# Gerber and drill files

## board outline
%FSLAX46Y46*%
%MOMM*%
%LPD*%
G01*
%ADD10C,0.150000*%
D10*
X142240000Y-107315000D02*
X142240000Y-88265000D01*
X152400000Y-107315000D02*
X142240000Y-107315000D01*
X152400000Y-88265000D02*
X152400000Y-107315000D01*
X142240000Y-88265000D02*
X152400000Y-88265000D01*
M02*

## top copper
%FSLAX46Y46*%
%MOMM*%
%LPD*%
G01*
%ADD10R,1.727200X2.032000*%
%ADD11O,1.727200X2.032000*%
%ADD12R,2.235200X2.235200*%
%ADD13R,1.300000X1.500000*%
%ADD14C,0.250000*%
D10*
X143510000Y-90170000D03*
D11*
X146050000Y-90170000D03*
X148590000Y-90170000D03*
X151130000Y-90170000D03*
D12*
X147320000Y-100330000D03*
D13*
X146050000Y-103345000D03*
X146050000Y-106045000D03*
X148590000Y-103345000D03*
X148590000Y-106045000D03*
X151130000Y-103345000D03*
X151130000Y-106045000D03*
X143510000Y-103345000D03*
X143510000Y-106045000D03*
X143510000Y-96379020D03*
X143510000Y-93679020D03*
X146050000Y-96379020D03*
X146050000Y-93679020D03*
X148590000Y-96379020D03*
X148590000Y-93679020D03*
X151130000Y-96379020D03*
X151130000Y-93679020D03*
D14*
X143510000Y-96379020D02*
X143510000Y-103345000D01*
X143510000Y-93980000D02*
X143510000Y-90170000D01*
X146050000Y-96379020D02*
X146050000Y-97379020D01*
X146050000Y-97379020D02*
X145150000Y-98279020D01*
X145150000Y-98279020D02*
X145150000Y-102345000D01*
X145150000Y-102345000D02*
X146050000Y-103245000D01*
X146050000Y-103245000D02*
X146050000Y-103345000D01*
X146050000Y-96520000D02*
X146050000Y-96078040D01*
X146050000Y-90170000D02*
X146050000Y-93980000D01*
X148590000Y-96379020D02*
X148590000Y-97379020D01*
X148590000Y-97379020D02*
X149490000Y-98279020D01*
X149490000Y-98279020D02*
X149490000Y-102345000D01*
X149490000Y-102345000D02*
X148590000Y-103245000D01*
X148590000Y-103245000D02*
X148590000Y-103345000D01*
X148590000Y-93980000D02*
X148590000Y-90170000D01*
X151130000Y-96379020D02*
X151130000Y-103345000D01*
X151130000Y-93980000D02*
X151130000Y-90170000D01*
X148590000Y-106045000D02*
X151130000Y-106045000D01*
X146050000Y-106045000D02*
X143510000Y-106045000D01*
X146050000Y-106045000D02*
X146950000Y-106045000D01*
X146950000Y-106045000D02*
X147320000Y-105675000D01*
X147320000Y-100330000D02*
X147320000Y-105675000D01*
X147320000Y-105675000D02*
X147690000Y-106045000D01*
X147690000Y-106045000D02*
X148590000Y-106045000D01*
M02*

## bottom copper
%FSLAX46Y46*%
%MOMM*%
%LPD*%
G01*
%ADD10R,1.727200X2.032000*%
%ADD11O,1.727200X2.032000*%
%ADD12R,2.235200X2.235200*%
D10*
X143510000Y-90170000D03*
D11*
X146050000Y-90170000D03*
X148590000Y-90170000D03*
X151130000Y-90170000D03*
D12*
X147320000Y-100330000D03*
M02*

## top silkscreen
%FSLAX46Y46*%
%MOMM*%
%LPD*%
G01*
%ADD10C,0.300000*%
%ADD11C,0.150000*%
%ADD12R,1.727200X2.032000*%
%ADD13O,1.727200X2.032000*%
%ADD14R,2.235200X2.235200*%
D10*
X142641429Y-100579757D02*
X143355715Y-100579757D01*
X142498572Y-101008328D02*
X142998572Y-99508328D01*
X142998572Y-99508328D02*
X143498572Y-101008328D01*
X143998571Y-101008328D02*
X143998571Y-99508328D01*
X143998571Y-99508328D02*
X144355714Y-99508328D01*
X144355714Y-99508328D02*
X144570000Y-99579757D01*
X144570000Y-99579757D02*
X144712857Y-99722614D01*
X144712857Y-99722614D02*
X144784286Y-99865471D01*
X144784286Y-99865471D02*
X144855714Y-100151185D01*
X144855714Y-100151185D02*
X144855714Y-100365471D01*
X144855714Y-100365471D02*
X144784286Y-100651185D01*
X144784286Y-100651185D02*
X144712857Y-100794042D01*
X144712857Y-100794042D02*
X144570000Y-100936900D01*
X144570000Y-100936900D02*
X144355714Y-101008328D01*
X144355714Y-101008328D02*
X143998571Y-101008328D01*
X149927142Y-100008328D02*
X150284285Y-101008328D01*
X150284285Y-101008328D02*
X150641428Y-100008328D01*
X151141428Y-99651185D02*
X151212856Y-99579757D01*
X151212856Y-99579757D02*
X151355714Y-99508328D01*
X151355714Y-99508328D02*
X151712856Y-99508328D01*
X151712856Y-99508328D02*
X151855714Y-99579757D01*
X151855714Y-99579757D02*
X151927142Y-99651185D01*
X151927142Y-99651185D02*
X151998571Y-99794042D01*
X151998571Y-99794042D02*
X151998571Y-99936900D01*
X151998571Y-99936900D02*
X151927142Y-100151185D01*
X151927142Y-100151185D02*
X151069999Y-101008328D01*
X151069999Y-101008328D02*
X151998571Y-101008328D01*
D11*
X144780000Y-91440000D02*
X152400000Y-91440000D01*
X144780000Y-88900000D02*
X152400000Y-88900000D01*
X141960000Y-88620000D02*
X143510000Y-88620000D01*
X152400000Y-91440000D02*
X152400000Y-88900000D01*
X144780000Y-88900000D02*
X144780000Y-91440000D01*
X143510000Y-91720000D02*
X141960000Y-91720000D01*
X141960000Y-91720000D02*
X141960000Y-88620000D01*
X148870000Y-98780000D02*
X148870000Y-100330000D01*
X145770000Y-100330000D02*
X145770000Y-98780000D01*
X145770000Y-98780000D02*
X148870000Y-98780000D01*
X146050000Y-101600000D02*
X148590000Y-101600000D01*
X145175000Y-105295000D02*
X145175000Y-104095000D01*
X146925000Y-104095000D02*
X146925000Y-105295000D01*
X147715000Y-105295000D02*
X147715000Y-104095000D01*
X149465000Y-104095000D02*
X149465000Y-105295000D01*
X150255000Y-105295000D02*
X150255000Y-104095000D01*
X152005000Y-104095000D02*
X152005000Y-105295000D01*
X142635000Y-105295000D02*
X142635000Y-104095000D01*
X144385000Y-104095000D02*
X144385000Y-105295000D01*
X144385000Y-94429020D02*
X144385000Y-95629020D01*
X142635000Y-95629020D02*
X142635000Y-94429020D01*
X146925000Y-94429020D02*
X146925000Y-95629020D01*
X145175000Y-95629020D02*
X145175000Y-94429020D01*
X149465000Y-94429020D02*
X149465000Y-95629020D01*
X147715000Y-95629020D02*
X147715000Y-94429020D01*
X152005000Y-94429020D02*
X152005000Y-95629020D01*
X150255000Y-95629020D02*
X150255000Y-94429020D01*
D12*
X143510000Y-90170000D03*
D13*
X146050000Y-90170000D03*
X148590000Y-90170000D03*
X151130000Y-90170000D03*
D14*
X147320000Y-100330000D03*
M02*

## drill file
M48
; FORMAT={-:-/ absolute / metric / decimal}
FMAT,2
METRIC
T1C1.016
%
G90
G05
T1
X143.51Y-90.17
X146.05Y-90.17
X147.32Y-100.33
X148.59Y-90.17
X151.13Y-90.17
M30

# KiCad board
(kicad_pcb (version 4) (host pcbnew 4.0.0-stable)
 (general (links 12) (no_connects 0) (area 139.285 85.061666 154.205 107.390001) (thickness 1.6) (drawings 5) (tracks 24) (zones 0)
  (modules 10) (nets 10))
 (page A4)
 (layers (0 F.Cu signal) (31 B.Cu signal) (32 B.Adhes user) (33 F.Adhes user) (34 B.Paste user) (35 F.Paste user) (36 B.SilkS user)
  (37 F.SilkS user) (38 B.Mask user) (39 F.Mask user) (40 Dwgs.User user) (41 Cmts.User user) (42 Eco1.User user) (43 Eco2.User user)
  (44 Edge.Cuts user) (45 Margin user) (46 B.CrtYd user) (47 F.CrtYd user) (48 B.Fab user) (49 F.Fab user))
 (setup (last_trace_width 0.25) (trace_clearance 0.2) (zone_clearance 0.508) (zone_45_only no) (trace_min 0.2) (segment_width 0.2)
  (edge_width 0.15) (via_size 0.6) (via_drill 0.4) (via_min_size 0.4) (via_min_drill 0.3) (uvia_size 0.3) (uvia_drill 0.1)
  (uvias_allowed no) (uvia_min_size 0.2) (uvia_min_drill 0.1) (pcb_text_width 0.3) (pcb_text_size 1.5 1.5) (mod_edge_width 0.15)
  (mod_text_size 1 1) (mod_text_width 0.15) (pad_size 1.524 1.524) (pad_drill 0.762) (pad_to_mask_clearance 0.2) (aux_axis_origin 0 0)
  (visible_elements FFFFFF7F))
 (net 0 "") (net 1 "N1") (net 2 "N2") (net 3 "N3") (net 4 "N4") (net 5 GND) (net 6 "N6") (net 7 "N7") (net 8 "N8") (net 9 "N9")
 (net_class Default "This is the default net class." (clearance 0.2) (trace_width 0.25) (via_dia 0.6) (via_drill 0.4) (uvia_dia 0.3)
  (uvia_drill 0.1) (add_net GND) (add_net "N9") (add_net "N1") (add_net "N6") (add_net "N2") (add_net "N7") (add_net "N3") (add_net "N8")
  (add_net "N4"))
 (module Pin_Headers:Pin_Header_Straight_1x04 (layer F.Cu) (at 143.51 90.17 90)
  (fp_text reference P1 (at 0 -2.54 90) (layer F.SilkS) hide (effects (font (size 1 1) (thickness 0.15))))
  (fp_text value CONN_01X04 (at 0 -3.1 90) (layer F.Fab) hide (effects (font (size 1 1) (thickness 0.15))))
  (fp_line (start -1.27 1.27) (end -1.27 8.89) (layer F.SilkS) (width 0.15))
  (fp_line (start 1.27 1.27) (end 1.27 8.89) (layer F.SilkS) (width 0.15))
  (fp_line (start 1.55 -1.55) (end 1.55 0) (layer F.SilkS) (width 0.15))
  (fp_line (start -1.27 8.89) (end 1.27 8.89) (layer F.SilkS) (width 0.15))
  (fp_line (start 1.27 1.27) (end -1.27 1.27) (layer F.SilkS) (width 0.15))
  (fp_line (start -1.55 0) (end -1.55 -1.55) (layer F.SilkS) (width 0.15))
  (fp_line (start -1.55 -1.55) (end 1.55 -1.55) (layer F.SilkS) (width 0.15))
  (pad 1 thru_hole rect (at 0 0 90) (size 2.032 1.7272) (drill 1.016) (layers *.Cu *.Mask F.SilkS) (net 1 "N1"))
  (pad 2 thru_hole oval (at 0 2.54 90) (size 2.032 1.7272) (drill 1.016) (layers *.Cu *.Mask F.SilkS) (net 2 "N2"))
  (pad 3 thru_hole oval (at 0 5.08 90) (size 2.032 1.7272) (drill 1.016) (layers *.Cu *.Mask F.SilkS) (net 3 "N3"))
  (pad 4 thru_hole oval (at 0 7.62 90) (size 2.032 1.7272) (drill 1.016) (layers *.Cu *.Mask F.SilkS) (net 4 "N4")))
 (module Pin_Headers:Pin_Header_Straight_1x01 (layer F.Cu) (at 147.32 100.33)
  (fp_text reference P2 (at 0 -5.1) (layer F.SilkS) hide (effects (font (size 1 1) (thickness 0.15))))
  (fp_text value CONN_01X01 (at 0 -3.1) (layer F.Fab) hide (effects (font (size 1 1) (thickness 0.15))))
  (fp_line (start 1.55 -1.55) (end 1.55 0) (layer F.SilkS) (width 0.15))
  (fp_line (start -1.55 0) (end -1.55 -1.55) (layer F.SilkS) (width 0.15))
  (fp_line (start -1.55 -1.55) (end 1.55 -1.55) (layer F.SilkS) (width 0.15))
  (fp_line (start -1.27 1.27) (end 1.27 1.27) (layer F.SilkS) (width 0.15))
  (pad 1 thru_hole rect (at 0 0) (size 2.2352 2.2352) (drill 1.016) (layers *.Cu *.Mask F.SilkS) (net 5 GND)))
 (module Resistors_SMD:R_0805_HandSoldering (layer F.Cu) (at 146.05 104.695 270)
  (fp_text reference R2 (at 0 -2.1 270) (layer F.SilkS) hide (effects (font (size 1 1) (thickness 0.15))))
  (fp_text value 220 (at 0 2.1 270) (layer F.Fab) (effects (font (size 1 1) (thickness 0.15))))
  (fp_line (start 0.6 0.875) (end -0.6 0.875) (layer F.SilkS) (width 0.15))
  (fp_line (start -0.6 -0.875) (end 0.6 -0.875) (layer F.SilkS) (width 0.15))
  (pad 1 smd rect (at -1.35 0 270) (size 1.5 1.3) (layers F.Cu F.Paste F.Mask) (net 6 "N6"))
  (pad 2 smd rect (at 1.35 0 270) (size 1.5 1.3) (layers F.Cu F.Paste F.Mask) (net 5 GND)))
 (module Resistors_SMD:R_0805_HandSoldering (layer F.Cu) (at 148.59 104.695 270)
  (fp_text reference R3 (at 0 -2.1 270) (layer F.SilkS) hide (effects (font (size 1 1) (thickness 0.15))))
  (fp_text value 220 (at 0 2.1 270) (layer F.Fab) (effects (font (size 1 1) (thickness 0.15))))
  (fp_line (start 0.6 0.875) (end -0.6 0.875) (layer F.SilkS) (width 0.15))
  (fp_line (start -0.6 -0.875) (end 0.6 -0.875) (layer F.SilkS) (width 0.15))
  (pad 1 smd rect (at -1.35 0 270) (size 1.5 1.3) (layers F.Cu F.Paste F.Mask) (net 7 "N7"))
  (pad 2 smd rect (at 1.35 0 270) (size 1.5 1.3) (layers F.Cu F.Paste F.Mask) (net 5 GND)))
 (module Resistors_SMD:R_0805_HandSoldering (layer F.Cu) (at 151.13 104.695 270)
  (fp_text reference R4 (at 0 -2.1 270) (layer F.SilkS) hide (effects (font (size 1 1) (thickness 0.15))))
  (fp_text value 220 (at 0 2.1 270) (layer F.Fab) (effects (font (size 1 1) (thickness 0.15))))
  (fp_line (start 0.6 0.875) (end -0.6 0.875) (layer F.SilkS) (width 0.15))
  (fp_line (start -0.6 -0.875) (end 0.6 -0.875) (layer F.SilkS) (width 0.15))
  (pad 1 smd rect (at -1.35 0 270) (size 1.5 1.3) (layers F.Cu F.Paste F.Mask) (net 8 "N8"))
  (pad 2 smd rect (at 1.35 0 270) (size 1.5 1.3) (layers F.Cu F.Paste F.Mask) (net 5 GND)))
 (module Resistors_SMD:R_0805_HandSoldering (layer F.Cu) (at 143.51 104.695 270)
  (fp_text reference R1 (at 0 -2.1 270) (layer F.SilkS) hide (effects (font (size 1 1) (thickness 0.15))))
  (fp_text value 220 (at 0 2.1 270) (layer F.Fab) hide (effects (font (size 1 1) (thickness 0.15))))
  (fp_line (start 0.6 0.875) (end -0.6 0.875) (layer F.SilkS) (width 0.15))
  (fp_line (start -0.6 -0.875) (end 0.6 -0.875) (layer F.SilkS) (width 0.15))
  (pad 1 smd rect (at -1.35 0 270) (size 1.5 1.3) (layers F.Cu F.Paste F.Mask) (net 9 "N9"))
  (pad 2 smd rect (at 1.35 0 270) (size 1.5 1.3) (layers F.Cu F.Paste F.Mask) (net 5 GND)))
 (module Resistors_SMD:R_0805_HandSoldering (layer F.Cu) (at 143.51 95.02902 90)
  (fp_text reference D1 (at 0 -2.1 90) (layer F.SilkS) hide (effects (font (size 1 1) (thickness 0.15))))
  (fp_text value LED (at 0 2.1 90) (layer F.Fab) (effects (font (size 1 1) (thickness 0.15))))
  (fp_line (start 0.6 0.875) (end -0.6 0.875) (layer F.SilkS) (width 0.15))
  (fp_line (start -0.6 -0.875) (end 0.6 -0.875) (layer F.SilkS) (width 0.15))
  (pad 1 smd rect (at -1.35 0 90) (size 1.5 1.3) (layers F.Cu F.Paste F.Mask) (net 9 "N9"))
  (pad 2 smd rect (at 1.35 0 90) (size 1.5 1.3) (layers F.Cu F.Paste F.Mask) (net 1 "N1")))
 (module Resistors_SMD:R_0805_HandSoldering (layer F.Cu) (at 146.05 95.02902 90)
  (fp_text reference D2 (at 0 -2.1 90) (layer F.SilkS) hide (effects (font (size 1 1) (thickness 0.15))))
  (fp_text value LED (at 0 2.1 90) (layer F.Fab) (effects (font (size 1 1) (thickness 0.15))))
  (fp_line (start 0.6 0.875) (end -0.6 0.875) (layer F.SilkS) (width 0.15))
  (fp_line (start -0.6 -0.875) (end 0.6 -0.875) (layer F.SilkS) (width 0.15))
  (pad 1 smd rect (at -1.35 0 90) (size 1.5 1.3) (layers F.Cu F.Paste F.Mask) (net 6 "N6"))
  (pad 2 smd rect (at 1.35 0 90) (size 1.5 1.3) (layers F.Cu F.Paste F.Mask) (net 2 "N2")))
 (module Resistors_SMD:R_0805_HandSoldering (layer F.Cu) (at 148.59 95.02902 90)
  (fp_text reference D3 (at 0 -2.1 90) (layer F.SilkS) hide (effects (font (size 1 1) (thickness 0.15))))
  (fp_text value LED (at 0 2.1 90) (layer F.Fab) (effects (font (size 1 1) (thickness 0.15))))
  (fp_line (start 0.6 0.875) (end -0.6 0.875) (layer F.SilkS) (width 0.15))
  (fp_line (start -0.6 -0.875) (end 0.6 -0.875) (layer F.SilkS) (width 0.15))
  (pad 1 smd rect (at -1.35 0 90) (size 1.5 1.3) (layers F.Cu F.Paste F.Mask) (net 7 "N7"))
  (pad 2 smd rect (at 1.35 0 90) (size 1.5 1.3) (layers F.Cu F.Paste F.Mask) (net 3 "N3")))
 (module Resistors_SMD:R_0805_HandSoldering (layer F.Cu) (at 151.13 95.02902 90)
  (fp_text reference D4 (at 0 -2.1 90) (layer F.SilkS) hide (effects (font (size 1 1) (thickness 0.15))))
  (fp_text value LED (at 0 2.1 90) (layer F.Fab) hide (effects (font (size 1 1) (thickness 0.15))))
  (fp_line (start 0.6 0.875) (end -0.6 0.875) (layer F.SilkS) (width 0.15))
  (fp_line (start -0.6 -0.875) (end 0.6 -0.875) (layer F.SilkS) (width 0.15))
  (pad 1 smd rect (at -1.35 0 90) (size 1.5 1.3) (layers F.Cu F.Paste F.Mask) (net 8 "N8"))
  (pad 2 smd rect (at 1.35 0 90) (size 1.5 1.3) (layers F.Cu F.Paste F.Mask) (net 4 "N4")))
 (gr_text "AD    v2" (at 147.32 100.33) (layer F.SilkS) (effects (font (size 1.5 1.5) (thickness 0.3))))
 (gr_line (start 142.24 107.315) (end 142.24 88.265) (angle 90) (layer Edge.Cuts) (width 0.15))
 (gr_line (start 152.4 107.315) (end 142.24 107.315) (angle 90) (layer Edge.Cuts) (width 0.15))
 (gr_line (start 152.4 88.265) (end 152.4 107.315) (angle 90) (layer Edge.Cuts) (width 0.15))
 (gr_line (start 142.24 88.265) (end 152.4 88.265) (angle 90) (layer Edge.Cuts) (width 0.15))
 (segment (start 143.51 96.37902) (end 143.51 103.345) (width 0.25) (layer F.Cu) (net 9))
 (segment (start 143.51 93.98) (end 143.51 90.17) (width 0.25) (layer F.Cu) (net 1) (status 30))
 (segment (start 146.05 96.37902) (end 146.05 97.37902) (width 0.25) (layer F.Cu) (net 6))
 (segment (start 146.05 97.37902) (end 145.15 98.27902) (width 0.25) (layer F.Cu) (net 6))
 (segment (start 145.15 98.27902) (end 145.15 102.345) (width 0.25) (layer F.Cu) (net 6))
 (segment (start 145.15 102.345) (end 146.05 103.245) (width 0.25) (layer F.Cu) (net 6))
 (segment (start 146.05 103.245) (end 146.05 103.345) (width 0.25) (layer F.Cu) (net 6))
 (segment (start 146.05 96.52) (end 146.05 96.07804) (width 0.25) (layer F.Cu) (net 6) (status 30))
 (segment (start 146.05 90.17) (end 146.05 93.98) (width 0.25) (layer F.Cu) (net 2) (status 30))
 (segment (start 148.59 96.37902) (end 148.59 97.37902) (width 0.25) (layer F.Cu) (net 7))
 (segment (start 148.59 97.37902) (end 149.49 98.27902) (width 0.25) (layer F.Cu) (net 7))
 (segment (start 149.49 98.27902) (end 149.49 102.345) (width 0.25) (layer F.Cu) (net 7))
 (segment (start 149.49 102.345) (end 148.59 103.245) (width 0.25) (layer F.Cu) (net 7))
 (segment (start 148.59 103.245) (end 148.59 103.345) (width 0.25) (layer F.Cu) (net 7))
 (segment (start 148.59 93.98) (end 148.59 90.17) (width 0.25) (layer F.Cu) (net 3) (status 30))
 (segment (start 151.13 96.37902) (end 151.13 103.345) (width 0.25) (layer F.Cu) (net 8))
 (segment (start 151.13 93.98) (end 151.13 90.17) (width 0.25) (layer F.Cu) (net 4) (status 30))
 (segment (start 148.59 106.045) (end 151.13 106.045) (width 0.25) (layer F.Cu) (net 5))
 (segment (start 146.05 106.045) (end 143.51 106.045) (width 0.25) (layer F.Cu) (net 5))
 (segment (start 146.05 106.045) (end 146.95 106.045) (width 0.25) (layer F.Cu) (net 5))
 (segment (start 146.95 106.045) (end 147.32 105.675) (width 0.25) (layer F.Cu) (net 5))
 (segment (start 147.32 100.33) (end 147.32 105.675) (width 0.25) (layer F.Cu) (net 5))
 (segment (start 147.32 105.675) (end 147.69 106.045) (width 0.25) (layer F.Cu) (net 5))
 (segment (start 147.69 106.045) (end 148.59 106.045) (width 0.25) (layer F.Cu) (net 5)))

